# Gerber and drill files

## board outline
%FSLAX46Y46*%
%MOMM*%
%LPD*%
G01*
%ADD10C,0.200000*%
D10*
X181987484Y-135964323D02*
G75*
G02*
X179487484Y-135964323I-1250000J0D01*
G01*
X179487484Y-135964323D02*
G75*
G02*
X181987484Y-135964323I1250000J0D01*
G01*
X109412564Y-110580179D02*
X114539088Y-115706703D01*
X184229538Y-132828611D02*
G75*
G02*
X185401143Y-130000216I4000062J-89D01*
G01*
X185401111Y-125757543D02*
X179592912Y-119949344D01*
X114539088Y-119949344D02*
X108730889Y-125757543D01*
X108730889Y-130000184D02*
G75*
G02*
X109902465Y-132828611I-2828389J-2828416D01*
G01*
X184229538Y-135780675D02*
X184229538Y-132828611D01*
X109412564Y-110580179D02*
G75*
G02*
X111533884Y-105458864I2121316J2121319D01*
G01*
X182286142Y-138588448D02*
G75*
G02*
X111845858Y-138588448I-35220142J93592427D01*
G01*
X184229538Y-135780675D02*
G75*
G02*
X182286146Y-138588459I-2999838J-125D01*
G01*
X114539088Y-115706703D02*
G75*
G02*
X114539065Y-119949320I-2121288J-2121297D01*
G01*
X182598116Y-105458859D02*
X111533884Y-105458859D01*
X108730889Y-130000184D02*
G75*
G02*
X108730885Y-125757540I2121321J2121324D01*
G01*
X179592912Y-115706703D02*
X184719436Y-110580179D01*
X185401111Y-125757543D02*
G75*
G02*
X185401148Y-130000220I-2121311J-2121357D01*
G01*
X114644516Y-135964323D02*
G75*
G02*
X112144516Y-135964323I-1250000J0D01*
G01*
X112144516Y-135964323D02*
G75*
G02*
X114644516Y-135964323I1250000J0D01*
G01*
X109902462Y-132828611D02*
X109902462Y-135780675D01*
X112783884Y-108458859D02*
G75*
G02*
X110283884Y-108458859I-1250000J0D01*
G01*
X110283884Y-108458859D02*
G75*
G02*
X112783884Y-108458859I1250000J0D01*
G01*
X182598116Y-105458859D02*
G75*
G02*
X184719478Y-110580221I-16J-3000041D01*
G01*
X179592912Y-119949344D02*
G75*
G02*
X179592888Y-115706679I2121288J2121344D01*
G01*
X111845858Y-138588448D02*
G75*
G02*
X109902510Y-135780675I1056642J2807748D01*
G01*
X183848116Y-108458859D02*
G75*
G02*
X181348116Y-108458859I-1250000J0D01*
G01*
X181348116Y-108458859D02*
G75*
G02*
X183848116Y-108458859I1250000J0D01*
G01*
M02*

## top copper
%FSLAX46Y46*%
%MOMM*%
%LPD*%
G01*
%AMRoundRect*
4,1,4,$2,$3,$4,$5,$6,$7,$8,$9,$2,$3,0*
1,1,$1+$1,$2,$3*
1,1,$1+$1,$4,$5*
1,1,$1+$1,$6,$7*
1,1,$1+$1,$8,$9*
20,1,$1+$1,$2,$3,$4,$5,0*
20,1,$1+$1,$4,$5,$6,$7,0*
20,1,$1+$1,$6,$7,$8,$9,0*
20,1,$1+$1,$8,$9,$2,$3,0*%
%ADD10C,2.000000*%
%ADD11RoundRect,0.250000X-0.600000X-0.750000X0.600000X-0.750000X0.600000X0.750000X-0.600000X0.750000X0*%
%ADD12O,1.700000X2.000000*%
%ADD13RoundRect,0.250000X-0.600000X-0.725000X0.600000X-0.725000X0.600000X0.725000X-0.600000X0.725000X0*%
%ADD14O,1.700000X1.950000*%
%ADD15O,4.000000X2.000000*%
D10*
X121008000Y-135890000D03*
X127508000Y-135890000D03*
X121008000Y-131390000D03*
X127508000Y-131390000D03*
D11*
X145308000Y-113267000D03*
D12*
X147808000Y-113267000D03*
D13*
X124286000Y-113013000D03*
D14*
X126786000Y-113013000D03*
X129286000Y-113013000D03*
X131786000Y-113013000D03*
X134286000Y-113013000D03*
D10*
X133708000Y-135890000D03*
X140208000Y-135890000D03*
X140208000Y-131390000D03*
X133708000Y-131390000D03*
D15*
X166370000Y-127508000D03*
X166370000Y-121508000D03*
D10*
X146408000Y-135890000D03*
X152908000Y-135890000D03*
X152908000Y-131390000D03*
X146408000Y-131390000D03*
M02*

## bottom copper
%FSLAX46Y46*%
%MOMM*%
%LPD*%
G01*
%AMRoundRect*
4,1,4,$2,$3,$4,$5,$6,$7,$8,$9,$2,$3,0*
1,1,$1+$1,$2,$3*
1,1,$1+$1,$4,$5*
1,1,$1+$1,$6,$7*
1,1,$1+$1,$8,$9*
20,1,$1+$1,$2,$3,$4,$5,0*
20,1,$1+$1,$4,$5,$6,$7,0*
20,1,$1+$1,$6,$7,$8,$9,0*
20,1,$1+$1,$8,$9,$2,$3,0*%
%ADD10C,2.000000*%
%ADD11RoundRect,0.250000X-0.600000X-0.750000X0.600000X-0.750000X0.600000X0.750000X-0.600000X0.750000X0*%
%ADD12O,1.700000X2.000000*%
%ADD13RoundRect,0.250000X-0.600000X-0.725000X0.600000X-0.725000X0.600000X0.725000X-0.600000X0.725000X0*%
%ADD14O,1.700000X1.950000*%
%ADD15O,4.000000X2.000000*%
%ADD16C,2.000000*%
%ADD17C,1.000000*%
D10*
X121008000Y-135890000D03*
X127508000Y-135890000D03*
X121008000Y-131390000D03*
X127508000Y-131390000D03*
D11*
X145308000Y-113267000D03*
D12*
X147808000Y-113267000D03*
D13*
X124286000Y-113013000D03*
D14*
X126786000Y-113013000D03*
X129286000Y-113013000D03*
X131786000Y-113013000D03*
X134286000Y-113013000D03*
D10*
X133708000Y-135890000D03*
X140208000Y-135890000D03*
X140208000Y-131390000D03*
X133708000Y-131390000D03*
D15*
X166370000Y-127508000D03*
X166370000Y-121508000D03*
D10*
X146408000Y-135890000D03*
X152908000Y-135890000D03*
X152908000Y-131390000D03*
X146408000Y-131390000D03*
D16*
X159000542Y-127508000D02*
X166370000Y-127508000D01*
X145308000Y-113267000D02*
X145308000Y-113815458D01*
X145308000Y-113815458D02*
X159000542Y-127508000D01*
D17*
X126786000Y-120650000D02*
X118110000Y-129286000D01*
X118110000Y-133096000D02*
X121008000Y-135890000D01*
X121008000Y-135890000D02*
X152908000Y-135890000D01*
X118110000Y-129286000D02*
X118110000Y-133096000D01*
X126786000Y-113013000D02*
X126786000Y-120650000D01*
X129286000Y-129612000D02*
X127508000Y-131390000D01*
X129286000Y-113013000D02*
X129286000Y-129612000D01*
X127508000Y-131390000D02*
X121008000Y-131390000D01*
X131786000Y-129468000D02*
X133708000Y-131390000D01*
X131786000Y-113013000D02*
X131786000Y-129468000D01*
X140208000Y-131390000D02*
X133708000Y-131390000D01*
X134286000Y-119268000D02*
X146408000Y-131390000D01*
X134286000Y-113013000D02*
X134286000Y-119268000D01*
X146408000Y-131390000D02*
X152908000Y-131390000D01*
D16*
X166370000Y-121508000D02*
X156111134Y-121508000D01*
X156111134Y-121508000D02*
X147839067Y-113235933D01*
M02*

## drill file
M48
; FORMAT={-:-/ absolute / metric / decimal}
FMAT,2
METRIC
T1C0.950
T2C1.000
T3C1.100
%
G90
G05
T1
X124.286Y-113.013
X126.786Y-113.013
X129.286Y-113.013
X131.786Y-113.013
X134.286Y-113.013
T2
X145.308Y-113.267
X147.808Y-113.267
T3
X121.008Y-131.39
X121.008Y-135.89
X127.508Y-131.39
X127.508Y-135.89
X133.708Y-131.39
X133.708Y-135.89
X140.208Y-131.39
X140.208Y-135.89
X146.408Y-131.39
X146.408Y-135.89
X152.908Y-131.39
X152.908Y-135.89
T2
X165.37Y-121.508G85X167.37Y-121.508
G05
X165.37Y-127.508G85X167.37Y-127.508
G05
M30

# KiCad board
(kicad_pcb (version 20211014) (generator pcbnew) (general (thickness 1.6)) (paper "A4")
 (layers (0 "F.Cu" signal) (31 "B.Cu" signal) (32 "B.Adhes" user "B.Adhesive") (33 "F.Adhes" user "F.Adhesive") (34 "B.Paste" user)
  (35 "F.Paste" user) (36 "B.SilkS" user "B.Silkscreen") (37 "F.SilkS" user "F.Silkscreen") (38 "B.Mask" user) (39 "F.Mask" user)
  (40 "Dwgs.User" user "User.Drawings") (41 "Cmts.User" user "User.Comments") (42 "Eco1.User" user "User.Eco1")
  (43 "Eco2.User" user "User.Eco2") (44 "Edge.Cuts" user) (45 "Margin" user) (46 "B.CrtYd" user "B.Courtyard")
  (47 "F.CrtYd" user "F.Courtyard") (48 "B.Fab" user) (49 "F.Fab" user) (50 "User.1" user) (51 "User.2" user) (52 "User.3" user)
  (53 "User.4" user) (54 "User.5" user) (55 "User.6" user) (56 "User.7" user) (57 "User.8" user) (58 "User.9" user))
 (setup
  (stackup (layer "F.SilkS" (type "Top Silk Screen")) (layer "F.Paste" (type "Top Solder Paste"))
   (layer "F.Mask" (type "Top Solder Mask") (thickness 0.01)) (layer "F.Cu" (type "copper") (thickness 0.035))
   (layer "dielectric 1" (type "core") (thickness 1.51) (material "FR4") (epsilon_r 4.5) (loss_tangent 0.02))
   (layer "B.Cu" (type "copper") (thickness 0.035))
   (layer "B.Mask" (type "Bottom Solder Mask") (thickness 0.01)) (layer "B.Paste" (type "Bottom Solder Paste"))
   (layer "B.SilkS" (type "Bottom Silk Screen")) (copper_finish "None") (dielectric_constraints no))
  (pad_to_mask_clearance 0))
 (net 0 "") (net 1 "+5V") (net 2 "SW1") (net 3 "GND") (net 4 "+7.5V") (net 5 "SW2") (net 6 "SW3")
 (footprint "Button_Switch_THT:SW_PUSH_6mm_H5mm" (layer "F.Cu") (at 127.508 135.89 180)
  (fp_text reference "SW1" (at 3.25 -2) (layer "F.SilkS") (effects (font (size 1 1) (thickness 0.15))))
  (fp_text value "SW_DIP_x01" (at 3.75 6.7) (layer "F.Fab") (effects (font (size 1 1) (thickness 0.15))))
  (pad "1" thru_hole circle (at 6.5 0 270) (size 2 2) (drill 1.1) (layers *.Cu *.Mask) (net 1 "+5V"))
  (pad "1" thru_hole circle (at 0 0 270) (size 2 2) (drill 1.1) (layers *.Cu *.Mask) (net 1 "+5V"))
  (pad "2" thru_hole circle (at 6.5 4.5 270) (size 2 2) (drill 1.1) (layers *.Cu *.Mask) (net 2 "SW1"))
  (pad "2" thru_hole circle (at 0 4.5 270) (size 2 2) (drill 1.1) (layers *.Cu *.Mask) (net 2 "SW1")))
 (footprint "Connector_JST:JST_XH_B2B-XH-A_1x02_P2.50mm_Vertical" (layer "F.Cu") (at 145.308 113.267)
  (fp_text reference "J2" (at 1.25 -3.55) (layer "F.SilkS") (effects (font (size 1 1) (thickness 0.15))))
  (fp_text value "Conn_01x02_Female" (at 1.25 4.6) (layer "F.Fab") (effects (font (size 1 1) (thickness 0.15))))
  (pad "1" thru_hole roundrect (at 0 0) (size 1.7 2) (drill 1) (layers *.Cu *.Mask) (roundrect_rratio 0.147059) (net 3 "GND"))
  (pad "2" thru_hole oval (at 2.5 0) (size 1.7 2) (drill 1) (layers *.Cu *.Mask) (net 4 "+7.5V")))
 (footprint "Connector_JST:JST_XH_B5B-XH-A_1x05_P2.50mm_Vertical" (layer "F.Cu") (at 124.286 113.013)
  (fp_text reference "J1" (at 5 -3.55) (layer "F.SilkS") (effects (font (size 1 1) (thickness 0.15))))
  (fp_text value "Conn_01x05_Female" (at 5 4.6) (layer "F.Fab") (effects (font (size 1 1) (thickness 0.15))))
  (pad "1" thru_hole roundrect (at 0 0) (size 1.7 1.95) (drill 0.95) (layers *.Cu *.Mask) (roundrect_rratio 0.147059) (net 3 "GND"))
  (pad "2" thru_hole oval (at 2.5 0) (size 1.7 1.95) (drill 0.95) (layers *.Cu *.Mask) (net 1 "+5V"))
  (pad "3" thru_hole oval (at 5 0) (size 1.7 1.95) (drill 0.95) (layers *.Cu *.Mask) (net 2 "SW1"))
  (pad "4" thru_hole oval (at 7.5 0) (size 1.7 1.95) (drill 0.95) (layers *.Cu *.Mask) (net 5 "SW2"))
  (pad "5" thru_hole oval (at 10 0) (size 1.7 1.95) (drill 0.95) (layers *.Cu *.Mask) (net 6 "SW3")))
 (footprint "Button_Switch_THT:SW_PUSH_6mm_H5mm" (layer "F.Cu") (at 140.208 135.89 180)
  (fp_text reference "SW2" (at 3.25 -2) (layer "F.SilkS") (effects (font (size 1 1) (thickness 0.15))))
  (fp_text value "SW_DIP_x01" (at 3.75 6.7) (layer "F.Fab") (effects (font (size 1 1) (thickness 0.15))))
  (pad "1" thru_hole circle (at 6.5 0 270) (size 2 2) (drill 1.1) (layers *.Cu *.Mask) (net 1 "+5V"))
  (pad "1" thru_hole circle (at 0 0 270) (size 2 2) (drill 1.1) (layers *.Cu *.Mask) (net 1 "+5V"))
  (pad "2" thru_hole circle (at 0 4.5 270) (size 2 2) (drill 1.1) (layers *.Cu *.Mask) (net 5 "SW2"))
  (pad "2" thru_hole circle (at 6.5 4.5 270) (size 2 2) (drill 1.1) (layers *.Cu *.Mask) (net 5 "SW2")))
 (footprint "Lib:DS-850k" (layer "F.Cu") (at 166.37 127.508 -90)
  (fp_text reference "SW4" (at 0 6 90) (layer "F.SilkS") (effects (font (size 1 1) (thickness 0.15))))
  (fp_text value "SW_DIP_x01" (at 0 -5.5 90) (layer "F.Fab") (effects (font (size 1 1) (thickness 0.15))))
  (pad "1" thru_hole oval locked (at 0 0) (size 4 2) (drill oval 3 1) (layers *.Cu *.Mask) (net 3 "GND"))
  (pad "2" thru_hole oval locked (at -6 0) (size 4 2) (drill oval 3 1) (layers *.Cu *.Mask) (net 4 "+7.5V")))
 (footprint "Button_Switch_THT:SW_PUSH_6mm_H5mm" (layer "F.Cu") (at 152.908 135.89 180)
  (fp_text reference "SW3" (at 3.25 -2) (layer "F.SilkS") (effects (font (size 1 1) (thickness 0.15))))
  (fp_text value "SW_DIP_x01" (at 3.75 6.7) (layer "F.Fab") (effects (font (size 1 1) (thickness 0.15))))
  (pad "1" thru_hole circle (at 6.5 0 270) (size 2 2) (drill 1.1) (layers *.Cu *.Mask) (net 1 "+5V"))
  (pad "1" thru_hole circle (at 0 0 270) (size 2 2) (drill 1.1) (layers *.Cu *.Mask) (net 1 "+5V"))
  (pad "2" thru_hole circle (at 0 4.5 270) (size 2 2) (drill 1.1) (layers *.Cu *.Mask) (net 6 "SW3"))
  (pad "2" thru_hole circle (at 6.5 4.5 270) (size 2 2) (drill 1.1) (layers *.Cu *.Mask) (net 6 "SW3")))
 (gr_circle (center 180.737484 135.964323) (end 181.987484 135.964323) (layer "Edge.Cuts") (width 0.2) (fill none))
 (gr_line (start 109.412564 110.580179) (end 114.539088 115.706703) (layer "Edge.Cuts") (width 0.2))
 (gr_arc (start 184.229538 132.828611) (mid 184.534027 131.297882) (end 185.401111 130.000184) (layer "Edge.Cuts") (width 0.2))
 (gr_line (start 185.401111 125.757543) (end 179.592912 119.949344) (layer "Edge.Cuts") (width 0.2))
 (gr_line (start 114.539088 119.949344) (end 108.730889 125.757543) (layer "Edge.Cuts") (width 0.2))
 (gr_arc (start 108.730889 130.000184) (mid 109.59798 131.297877) (end 109.902462 132.828611) (layer "Edge.Cuts") (width 0.2))
 (gr_line (start 184.229538 135.780675) (end 184.229538 132.828611) (layer "Edge.Cuts") (width 0.2))
 (gr_arc (start 109.412564 110.580179) (mid 108.762246 107.310809) (end 111.533884 105.458859) (layer "Edge.Cuts") (width 0.2))
 (gr_arc (start 182.286142 138.588448) (mid 147.066 144.996025) (end 111.845858 138.588448) (layer "Edge.Cuts") (width 0.2))
 (gr_arc (start 184.229538 135.780675) (mid 183.696321 137.488069) (end 182.286142 138.588448) (layer "Edge.Cuts") (width 0.2))
 (gr_arc (start 114.539088 115.706703) (mid 115.417768 117.828024) (end 114.539088 119.949344) (layer "Edge.Cuts") (width 0.2))
 (gr_line (start 182.598116 105.458859) (end 111.533884 105.458859) (layer "Edge.Cuts") (width 0.2))
 (gr_arc (start 108.730889 130.000184) (mid 107.852209 127.878864) (end 108.730889 125.757543) (layer "Edge.Cuts") (width 0.2))
 (gr_line (start 179.592912 115.706703) (end 184.719436 110.580179) (layer "Edge.Cuts") (width 0.2))
 (gr_arc (start 185.401111 125.757543) (mid 186.279792 127.878864) (end 185.401111 130.000184) (layer "Edge.Cuts") (width 0.2))
 (gr_circle (center 113.394516 135.964323) (end 114.644516 135.964323) (layer "Edge.Cuts") (width 0.2) (fill none))
 (gr_line (start 109.902462 132.828611) (end 109.902462 135.780675) (layer "Edge.Cuts") (width 0.2))
 (gr_circle (center 111.533884 108.458859) (end 112.783884 108.458859) (layer "Edge.Cuts") (width 0.2) (fill none))
 (gr_arc (start 182.598116 105.458859) (mid 185.369755 107.310807) (end 184.719436 110.580179) (layer "Edge.Cuts") (width 0.2))
 (gr_arc (start 179.592912 119.949344) (mid 178.714233 117.828024) (end 179.592912 115.706703) (layer "Edge.Cuts") (width 0.2))
 (gr_arc (start 111.845858 138.588448) (mid 110.435702 137.48804) (end 109.902462 135.780675) (layer "Edge.Cuts") (width 0.2))
 (gr_circle (center 182.598116 108.458859) (end 183.848116 108.458859) (layer "Edge.Cuts") (width 0.2) (fill none))
 (segment (start 159.000542 127.508) (end 166.37 127.508) (width 2) (layer "B.Cu") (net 3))
 (segment (start 145.308 113.267) (end 145.308 113.815458) (width 2) (layer "B.Cu") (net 3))
 (segment (start 145.308 113.815458) (end 159.000542 127.508) (width 2) (layer "B.Cu") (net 3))
 (segment (start 126.786 120.65) (end 118.11 129.286) (width 1) (layer "B.Cu") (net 1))
 (segment (start 118.11 133.096) (end 121.008 135.89) (width 1) (layer "B.Cu") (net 1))
 (segment (start 121.008 135.89) (end 152.908 135.89) (width 1) (layer "B.Cu") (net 1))
 (segment (start 118.11 129.286) (end 118.11 133.096) (width 1) (layer "B.Cu") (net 1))
 (segment (start 126.786 113.013) (end 126.786 120.65) (width 1) (layer "B.Cu") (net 1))
 (segment (start 129.286 129.612) (end 127.508 131.39) (width 1) (layer "B.Cu") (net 2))
 (segment (start 129.286 113.013) (end 129.286 129.612) (width 1) (layer "B.Cu") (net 2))
 (segment (start 127.508 131.39) (end 121.008 131.39) (width 1) (layer "B.Cu") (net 2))
 (segment (start 131.786 129.468) (end 133.708 131.39) (width 1) (layer "B.Cu") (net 5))
 (segment (start 131.786 113.013) (end 131.786 129.468) (width 1) (layer "B.Cu") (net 5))
 (segment (start 140.208 131.39) (end 133.708 131.39) (width 1) (layer "B.Cu") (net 5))
 (segment (start 134.286 119.268) (end 146.408 131.39) (width 1) (layer "B.Cu") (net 6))
 (segment (start 134.286 113.013) (end 134.286 119.268) (width 1) (layer "B.Cu") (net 6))
 (segment (start 146.408 131.39) (end 152.908 131.39) (width 1) (layer "B.Cu") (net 6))
 (segment (start 166.37 121.508) (end 156.111134 121.508) (width 2) (layer "B.Cu") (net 4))
 (segment (start 156.111134 121.508) (end 147.839067 113.235933) (width 2) (layer "B.Cu") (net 4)))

